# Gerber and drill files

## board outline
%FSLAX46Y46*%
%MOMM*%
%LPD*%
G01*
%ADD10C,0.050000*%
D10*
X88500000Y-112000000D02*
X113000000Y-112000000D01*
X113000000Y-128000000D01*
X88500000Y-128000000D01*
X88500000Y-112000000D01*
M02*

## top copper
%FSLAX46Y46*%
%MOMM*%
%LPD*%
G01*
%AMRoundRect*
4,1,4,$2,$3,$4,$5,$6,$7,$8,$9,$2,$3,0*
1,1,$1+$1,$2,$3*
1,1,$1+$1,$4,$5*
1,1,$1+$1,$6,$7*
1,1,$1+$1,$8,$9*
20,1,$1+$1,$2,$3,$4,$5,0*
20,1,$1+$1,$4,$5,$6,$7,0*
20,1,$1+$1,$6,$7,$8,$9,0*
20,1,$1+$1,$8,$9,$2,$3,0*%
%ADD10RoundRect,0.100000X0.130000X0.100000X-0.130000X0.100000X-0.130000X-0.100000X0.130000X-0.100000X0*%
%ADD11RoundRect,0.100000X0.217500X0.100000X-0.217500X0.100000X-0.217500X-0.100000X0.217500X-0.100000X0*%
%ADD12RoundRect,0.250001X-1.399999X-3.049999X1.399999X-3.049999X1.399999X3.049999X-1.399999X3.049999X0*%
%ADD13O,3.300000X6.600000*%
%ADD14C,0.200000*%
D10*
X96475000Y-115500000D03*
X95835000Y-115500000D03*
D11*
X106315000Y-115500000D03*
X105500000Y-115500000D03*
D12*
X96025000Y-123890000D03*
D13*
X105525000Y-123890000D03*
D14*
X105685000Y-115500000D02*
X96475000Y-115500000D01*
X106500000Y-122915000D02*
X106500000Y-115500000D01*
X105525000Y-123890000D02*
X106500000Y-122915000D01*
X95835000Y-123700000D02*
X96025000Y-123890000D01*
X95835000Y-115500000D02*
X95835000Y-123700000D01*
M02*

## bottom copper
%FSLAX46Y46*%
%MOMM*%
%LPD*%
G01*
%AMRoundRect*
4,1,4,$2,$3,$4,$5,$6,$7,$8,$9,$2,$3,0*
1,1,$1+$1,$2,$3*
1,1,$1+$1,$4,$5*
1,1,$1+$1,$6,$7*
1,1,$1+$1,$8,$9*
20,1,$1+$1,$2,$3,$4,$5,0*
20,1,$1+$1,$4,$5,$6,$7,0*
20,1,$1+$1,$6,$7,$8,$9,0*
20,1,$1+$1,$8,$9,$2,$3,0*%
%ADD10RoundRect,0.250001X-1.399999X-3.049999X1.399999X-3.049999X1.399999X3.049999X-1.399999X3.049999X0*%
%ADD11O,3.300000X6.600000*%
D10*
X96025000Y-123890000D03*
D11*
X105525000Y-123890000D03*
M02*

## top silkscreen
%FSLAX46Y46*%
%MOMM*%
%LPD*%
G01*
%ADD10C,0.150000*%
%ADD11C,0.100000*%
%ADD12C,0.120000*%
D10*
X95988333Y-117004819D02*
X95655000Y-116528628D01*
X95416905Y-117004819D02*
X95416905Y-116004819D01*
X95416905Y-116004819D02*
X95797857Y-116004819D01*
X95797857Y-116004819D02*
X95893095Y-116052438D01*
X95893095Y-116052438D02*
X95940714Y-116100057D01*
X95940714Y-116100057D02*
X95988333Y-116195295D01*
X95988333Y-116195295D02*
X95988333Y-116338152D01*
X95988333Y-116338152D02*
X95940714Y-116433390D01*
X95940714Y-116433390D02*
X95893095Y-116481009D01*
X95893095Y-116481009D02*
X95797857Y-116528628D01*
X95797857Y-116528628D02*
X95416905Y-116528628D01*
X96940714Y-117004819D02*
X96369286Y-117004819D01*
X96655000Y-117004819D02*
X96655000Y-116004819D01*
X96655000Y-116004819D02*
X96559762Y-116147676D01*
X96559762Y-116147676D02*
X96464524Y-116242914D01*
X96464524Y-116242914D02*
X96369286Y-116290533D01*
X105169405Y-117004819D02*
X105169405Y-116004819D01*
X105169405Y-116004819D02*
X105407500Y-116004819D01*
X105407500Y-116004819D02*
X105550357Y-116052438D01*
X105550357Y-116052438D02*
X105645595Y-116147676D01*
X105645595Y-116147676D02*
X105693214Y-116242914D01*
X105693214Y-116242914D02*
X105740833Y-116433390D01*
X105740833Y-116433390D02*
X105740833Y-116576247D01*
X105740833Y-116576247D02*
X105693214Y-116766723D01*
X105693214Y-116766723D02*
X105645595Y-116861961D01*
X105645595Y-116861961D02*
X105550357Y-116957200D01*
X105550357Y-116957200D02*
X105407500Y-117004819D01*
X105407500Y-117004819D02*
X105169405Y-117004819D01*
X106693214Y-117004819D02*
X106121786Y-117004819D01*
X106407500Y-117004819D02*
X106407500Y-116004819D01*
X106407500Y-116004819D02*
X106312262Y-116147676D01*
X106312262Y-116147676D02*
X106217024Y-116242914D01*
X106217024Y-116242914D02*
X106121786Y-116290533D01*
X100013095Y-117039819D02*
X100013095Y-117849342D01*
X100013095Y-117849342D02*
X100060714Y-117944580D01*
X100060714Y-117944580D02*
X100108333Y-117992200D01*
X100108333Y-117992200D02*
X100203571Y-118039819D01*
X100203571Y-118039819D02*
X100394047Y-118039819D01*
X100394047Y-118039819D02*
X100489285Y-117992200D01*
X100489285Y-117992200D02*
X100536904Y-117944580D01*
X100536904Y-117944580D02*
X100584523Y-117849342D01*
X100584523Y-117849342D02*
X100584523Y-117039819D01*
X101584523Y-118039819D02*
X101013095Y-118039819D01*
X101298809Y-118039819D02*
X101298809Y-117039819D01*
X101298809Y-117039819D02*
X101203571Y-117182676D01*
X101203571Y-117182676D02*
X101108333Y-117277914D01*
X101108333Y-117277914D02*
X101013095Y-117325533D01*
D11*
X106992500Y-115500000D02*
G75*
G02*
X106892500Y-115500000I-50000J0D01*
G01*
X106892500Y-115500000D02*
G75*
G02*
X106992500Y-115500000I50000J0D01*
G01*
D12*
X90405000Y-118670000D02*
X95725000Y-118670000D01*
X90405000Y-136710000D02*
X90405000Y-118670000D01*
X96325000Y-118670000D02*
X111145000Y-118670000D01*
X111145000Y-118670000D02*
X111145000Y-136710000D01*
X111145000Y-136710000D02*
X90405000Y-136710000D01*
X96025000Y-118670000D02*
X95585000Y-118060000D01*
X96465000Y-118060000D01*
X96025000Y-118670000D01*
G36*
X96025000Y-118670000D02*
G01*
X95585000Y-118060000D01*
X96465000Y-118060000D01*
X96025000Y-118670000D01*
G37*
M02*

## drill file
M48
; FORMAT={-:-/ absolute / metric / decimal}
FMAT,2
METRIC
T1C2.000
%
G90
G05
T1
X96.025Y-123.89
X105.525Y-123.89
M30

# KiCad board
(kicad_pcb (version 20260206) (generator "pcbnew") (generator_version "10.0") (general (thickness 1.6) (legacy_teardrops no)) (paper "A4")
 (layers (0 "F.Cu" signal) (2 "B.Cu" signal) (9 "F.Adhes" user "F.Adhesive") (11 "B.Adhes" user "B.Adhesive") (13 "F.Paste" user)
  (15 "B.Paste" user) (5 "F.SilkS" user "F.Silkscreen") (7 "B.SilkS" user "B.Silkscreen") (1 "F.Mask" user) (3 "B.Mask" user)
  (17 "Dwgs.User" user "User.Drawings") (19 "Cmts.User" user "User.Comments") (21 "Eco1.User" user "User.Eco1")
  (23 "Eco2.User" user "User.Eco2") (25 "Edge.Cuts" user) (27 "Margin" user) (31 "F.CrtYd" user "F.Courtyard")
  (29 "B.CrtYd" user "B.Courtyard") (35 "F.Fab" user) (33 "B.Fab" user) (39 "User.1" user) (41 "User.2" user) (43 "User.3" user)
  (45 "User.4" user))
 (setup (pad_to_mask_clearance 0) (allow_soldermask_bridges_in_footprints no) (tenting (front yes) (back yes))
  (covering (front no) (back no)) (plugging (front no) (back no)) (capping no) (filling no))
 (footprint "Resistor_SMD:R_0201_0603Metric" (layer "F.Cu") (at 96.155 115.5 180)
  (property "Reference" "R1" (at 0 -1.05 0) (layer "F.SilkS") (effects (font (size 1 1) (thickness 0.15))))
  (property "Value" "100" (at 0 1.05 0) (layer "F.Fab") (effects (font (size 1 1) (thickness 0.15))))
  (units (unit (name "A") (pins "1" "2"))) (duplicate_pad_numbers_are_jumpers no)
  (pad "" smd roundrect (at -0.345 0 180) (size 0.318 0.36) (layers "F.Paste") (roundrect_rratio 0.25))
  (pad "" smd roundrect (at 0.345 0 180) (size 0.318 0.36) (layers "F.Paste") (roundrect_rratio 0.25))
  (pad "1" smd roundrect (at -0.32 0 180) (size 0.46 0.4) (layers "F.Cu" "F.Mask") (roundrect_rratio 0.25) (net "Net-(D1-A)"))
  (pad "2" smd roundrect (at 0.32 0 180) (size 0.46 0.4) (layers "F.Cu" "F.Mask") (roundrect_rratio 0.25) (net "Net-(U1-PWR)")))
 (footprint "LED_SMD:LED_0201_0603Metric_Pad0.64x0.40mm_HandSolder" (layer "F.Cu") (at 105.9075 115.5 180)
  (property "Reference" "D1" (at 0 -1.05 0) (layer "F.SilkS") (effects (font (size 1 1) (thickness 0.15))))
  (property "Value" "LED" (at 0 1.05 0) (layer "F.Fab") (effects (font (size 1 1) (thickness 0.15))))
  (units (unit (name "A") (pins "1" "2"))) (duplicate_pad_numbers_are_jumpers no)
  (fp_circle (center -1.035 0) (end -0.985 0) (stroke (width 0.1) (type solid)) (fill no) (layer "F.SilkS"))
  (pad "" smd roundrect (at -0.4325 0 180) (size 0.458 0.36) (layers "F.Paste") (roundrect_rratio 0.25))
  (pad "" smd roundrect (at 0.4325 0 180) (size 0.458 0.36) (layers "F.Paste") (roundrect_rratio 0.25))
  (pad "1" smd roundrect (at -0.4075 0 180) (size 0.635 0.4) (layers "F.Cu" "F.Mask") (roundrect_rratio 0.25) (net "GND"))
  (pad "2" smd roundrect (at 0.4075 0 180) (size 0.635 0.4) (layers "F.Cu" "F.Mask") (roundrect_rratio 0.25) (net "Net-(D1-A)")))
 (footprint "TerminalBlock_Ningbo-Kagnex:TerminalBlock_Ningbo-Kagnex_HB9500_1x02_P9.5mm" (layer "F.Cu") (at 96.025 123.89)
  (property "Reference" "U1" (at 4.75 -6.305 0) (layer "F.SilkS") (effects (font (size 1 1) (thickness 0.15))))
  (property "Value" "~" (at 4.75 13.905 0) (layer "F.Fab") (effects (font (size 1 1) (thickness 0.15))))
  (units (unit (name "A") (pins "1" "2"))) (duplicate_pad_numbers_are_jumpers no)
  (fp_line (start -5.62 -5.22) (end -0.3 -5.22) (stroke (width 0.12) (type solid)) (layer "F.SilkS"))
  (fp_line (start -5.62 12.82) (end -5.62 -5.22) (stroke (width 0.12) (type solid)) (layer "F.SilkS"))
  (fp_line (start 0.3 -5.22) (end 15.12 -5.22) (stroke (width 0.12) (type solid)) (layer "F.SilkS"))
  (fp_line (start 15.12 -5.22) (end 15.12 12.82) (stroke (width 0.12) (type solid)) (layer "F.SilkS"))
  (fp_line (start 15.12 12.82) (end -5.62 12.82) (stroke (width 0.12) (type solid)) (layer "F.SilkS"))
  (fp_poly (pts (xy 0 -5.22) (xy -0.44 -5.83) (xy 0.44 -5.83)) (stroke (width 0.12) (type solid)) (fill yes) (layer "F.SilkS"))
  (pad "1" thru_hole roundrect (at 0 0) (size 3.3 6.6) (drill 2) (layers "*.Cu" "*.Mask") (remove_unused_layers no)
   (roundrect_rratio 0.075758) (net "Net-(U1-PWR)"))
  (pad "2" thru_hole oval (at 9.5 0) (size 3.3 6.6) (drill 2) (layers "*.Cu" "*.Mask") (remove_unused_layers no) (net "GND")))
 (gr_rect (start 88.5 112) (end 113 128) (stroke (width 0.05) (type default)) (fill no) (layer "Edge.Cuts"))
 (segment (start 105.685 115.5) (end 96.475 115.5) (width 0.2) (layer "F.Cu") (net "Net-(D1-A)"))
 (segment (start 106.5 122.915) (end 106.5 115.5) (width 0.2) (layer "F.Cu") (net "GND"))
 (segment (start 105.525 123.89) (end 106.5 122.915) (width 0.2) (layer "F.Cu") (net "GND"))
 (segment (start 95.835 123.7) (end 96.025 123.89) (width 0.2) (layer "F.Cu") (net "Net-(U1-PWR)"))
 (segment (start 95.835 115.5) (end 95.835 123.7) (width 0.2) (layer "F.Cu") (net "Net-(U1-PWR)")))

